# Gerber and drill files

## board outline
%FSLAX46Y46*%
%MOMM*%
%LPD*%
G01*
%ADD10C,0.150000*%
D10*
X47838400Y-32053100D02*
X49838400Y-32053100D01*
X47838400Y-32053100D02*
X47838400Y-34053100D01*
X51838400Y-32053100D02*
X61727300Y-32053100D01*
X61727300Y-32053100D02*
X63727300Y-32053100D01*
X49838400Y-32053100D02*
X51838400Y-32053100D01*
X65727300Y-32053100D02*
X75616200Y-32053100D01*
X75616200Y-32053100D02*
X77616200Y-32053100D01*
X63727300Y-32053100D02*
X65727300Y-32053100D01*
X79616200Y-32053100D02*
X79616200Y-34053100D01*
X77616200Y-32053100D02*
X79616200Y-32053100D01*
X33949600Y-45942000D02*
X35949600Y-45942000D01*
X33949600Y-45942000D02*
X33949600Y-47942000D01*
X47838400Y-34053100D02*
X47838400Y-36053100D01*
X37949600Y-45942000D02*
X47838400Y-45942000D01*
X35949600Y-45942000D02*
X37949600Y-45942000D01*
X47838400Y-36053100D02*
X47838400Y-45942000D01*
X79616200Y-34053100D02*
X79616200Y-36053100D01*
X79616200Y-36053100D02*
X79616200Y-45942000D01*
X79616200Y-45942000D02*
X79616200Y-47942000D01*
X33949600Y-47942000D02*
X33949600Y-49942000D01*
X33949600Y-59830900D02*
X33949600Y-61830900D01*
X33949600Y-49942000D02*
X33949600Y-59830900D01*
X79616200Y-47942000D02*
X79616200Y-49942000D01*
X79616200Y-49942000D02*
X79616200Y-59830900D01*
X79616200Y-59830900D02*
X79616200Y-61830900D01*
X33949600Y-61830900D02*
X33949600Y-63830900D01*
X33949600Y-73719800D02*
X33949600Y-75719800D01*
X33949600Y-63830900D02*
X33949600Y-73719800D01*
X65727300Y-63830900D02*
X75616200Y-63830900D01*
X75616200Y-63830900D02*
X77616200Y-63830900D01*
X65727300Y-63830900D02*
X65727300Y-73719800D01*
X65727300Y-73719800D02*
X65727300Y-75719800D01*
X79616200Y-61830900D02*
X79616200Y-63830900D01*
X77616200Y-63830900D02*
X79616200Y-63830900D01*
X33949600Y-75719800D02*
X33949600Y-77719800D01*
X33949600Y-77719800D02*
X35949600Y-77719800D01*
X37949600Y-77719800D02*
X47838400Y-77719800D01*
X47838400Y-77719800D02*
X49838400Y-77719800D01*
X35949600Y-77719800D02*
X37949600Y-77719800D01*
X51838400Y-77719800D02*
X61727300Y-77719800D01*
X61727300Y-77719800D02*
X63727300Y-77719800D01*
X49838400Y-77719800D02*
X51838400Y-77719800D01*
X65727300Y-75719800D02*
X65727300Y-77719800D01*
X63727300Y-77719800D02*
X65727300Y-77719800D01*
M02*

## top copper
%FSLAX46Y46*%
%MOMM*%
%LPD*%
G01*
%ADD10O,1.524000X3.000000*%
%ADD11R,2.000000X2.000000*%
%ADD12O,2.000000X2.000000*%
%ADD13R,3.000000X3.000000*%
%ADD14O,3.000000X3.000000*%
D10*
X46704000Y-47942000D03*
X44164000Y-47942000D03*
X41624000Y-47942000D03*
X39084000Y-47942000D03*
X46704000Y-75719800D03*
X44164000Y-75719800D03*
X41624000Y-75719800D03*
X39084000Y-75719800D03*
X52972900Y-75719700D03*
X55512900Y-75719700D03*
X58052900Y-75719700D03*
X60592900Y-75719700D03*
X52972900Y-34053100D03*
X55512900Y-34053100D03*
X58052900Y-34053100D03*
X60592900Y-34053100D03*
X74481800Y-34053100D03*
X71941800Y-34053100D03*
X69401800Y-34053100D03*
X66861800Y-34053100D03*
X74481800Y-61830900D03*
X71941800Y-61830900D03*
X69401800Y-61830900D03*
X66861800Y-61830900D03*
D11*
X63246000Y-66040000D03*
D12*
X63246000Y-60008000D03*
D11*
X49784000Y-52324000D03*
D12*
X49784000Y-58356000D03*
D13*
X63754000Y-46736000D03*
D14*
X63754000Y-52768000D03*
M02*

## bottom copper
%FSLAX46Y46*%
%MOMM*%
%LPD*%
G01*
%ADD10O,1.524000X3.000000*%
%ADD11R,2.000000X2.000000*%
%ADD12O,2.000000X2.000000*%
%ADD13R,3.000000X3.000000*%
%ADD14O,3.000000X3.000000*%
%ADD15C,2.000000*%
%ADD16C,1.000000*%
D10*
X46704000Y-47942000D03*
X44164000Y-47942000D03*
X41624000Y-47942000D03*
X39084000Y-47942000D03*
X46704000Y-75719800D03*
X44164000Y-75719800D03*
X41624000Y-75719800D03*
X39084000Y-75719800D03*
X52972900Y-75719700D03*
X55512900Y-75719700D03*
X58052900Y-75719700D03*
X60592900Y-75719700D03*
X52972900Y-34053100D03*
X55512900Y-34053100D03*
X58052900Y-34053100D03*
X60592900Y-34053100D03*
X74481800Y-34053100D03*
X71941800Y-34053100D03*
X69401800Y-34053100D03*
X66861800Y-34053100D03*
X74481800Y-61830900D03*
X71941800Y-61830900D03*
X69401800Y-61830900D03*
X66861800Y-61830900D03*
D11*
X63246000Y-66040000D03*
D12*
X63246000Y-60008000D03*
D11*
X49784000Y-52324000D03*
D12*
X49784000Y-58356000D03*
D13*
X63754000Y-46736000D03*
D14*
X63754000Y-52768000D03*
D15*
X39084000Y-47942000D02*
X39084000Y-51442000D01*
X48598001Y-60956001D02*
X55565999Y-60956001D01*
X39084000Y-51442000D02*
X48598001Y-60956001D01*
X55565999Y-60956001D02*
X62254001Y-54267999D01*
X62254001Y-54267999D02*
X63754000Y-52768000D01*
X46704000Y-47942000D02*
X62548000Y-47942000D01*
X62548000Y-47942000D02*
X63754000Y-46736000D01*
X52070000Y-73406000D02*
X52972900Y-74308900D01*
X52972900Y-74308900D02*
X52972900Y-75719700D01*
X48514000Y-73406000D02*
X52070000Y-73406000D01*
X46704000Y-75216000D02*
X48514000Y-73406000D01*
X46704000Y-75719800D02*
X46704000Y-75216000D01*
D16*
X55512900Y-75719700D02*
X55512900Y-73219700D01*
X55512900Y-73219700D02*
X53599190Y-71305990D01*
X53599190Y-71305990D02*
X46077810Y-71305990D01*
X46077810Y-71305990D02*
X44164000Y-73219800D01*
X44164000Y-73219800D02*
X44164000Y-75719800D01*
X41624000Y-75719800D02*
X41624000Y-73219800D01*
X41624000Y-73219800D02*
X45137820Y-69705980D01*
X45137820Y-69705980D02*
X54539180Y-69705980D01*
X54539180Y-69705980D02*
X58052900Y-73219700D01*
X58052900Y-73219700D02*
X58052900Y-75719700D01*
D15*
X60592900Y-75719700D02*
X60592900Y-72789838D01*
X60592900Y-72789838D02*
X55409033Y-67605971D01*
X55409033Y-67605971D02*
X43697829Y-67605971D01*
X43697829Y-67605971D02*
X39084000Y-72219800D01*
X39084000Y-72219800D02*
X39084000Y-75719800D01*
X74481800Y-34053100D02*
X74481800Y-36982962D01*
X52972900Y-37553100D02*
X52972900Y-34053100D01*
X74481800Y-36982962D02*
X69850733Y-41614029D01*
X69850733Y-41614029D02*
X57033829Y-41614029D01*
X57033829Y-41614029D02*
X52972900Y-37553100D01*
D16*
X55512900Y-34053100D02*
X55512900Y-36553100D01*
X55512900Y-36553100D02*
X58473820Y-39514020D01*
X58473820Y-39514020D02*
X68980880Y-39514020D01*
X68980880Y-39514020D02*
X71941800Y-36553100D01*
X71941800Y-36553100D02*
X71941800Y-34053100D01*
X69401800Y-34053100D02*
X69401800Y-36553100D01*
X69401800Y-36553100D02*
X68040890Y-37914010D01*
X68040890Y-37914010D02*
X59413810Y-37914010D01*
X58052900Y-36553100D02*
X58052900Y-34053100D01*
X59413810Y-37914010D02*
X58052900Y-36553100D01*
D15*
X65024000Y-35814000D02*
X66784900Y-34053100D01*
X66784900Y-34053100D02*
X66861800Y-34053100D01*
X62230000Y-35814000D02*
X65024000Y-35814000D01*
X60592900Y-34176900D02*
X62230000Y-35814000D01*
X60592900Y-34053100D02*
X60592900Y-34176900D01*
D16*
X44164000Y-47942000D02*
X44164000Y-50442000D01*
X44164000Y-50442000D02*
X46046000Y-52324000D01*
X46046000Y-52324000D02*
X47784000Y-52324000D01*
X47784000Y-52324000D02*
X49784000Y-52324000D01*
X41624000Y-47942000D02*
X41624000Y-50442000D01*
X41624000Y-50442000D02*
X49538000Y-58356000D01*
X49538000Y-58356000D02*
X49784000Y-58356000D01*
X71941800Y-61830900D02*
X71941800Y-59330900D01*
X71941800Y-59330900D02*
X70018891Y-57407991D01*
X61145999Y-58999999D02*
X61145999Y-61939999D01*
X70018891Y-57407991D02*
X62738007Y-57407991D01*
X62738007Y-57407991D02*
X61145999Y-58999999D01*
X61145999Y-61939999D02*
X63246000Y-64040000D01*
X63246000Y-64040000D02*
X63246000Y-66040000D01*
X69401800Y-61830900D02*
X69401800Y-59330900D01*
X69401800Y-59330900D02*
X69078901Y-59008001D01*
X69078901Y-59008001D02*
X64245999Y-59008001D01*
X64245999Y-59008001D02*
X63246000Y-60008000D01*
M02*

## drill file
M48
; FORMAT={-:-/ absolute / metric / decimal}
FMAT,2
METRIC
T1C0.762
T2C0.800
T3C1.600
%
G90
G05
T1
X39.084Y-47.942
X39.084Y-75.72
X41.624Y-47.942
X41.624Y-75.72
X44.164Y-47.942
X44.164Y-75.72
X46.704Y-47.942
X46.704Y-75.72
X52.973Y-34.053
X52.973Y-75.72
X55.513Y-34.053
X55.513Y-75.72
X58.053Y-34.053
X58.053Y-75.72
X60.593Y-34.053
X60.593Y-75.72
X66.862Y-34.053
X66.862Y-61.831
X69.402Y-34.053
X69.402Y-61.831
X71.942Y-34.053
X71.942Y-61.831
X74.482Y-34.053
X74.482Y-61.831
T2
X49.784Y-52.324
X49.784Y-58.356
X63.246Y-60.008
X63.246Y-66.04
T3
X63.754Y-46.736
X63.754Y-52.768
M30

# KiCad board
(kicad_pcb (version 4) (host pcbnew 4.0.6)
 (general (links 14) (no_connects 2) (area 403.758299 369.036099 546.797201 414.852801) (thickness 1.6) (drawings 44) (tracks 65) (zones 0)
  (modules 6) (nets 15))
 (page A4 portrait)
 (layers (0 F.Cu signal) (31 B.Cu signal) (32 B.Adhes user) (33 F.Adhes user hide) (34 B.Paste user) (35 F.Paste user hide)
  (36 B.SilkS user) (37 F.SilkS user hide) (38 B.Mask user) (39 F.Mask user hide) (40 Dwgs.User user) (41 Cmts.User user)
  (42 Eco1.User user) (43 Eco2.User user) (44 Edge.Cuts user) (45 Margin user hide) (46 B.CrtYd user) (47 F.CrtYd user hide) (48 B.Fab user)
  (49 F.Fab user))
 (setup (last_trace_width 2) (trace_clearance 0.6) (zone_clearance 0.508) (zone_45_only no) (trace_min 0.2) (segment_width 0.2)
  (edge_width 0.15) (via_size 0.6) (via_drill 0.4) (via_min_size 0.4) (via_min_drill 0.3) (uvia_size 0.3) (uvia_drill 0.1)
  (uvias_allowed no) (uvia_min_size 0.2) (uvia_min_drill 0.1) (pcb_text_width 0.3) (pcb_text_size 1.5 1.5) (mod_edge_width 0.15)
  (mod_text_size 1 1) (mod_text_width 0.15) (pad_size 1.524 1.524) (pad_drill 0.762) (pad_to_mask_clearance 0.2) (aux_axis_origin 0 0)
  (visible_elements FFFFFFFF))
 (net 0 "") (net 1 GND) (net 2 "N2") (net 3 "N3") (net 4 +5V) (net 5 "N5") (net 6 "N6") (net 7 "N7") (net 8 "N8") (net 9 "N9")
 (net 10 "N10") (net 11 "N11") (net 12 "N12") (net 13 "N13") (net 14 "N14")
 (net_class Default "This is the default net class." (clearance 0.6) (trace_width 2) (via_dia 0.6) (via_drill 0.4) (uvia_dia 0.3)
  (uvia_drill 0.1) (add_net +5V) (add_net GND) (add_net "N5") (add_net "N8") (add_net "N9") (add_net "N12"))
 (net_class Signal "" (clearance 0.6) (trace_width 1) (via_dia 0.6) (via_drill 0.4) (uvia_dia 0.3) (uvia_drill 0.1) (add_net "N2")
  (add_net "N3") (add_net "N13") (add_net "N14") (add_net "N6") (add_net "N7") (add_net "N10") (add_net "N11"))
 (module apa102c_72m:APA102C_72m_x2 (layer B.Cu) (at 42.894 61.8309 270)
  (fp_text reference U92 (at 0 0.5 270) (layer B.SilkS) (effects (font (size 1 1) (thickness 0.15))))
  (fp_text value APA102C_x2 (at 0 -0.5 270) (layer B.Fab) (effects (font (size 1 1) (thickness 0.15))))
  (pad 1 thru_hole oval (at -13.8889 -3.81 270) (size 3 1.524) (drill 0.762) (layers *.Cu *.Mask) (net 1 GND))
  (pad 2 thru_hole oval (at -13.8889 -1.27 270) (size 3 1.524) (drill 0.762) (layers *.Cu *.Mask) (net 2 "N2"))
  (pad 3 thru_hole oval (at -13.8889 1.27 270) (size 3 1.524) (drill 0.762) (layers *.Cu *.Mask) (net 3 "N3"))
  (pad 4 thru_hole oval (at -13.8889 3.81 270) (size 3 1.524) (drill 0.762) (layers *.Cu *.Mask) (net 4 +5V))
  (pad 5 thru_hole oval (at 13.8889 -3.81 270) (size 3 1.524) (drill 0.762) (layers *.Cu *.Mask) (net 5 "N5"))
  (pad 6 thru_hole oval (at 13.8889 -1.27 270) (size 3 1.524) (drill 0.762) (layers *.Cu *.Mask) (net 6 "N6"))
  (pad 7 thru_hole oval (at 13.8889 1.27 270) (size 3 1.524) (drill 0.762) (layers *.Cu *.Mask) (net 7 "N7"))
  (pad 8 thru_hole oval (at 13.8889 3.81 270) (size 3 1.524) (drill 0.762) (layers *.Cu *.Mask) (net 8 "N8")))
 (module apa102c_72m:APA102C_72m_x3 (layer B.Cu) (at 56.7829 54.8864 90)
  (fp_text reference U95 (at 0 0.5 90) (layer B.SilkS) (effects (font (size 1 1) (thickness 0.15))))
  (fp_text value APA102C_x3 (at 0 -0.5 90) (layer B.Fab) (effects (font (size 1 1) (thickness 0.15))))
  (pad 1 thru_hole oval (at -20.8333 -3.81 90) (size 3 1.524) (drill 0.762) (layers *.Cu *.Mask) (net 5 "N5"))
  (pad 2 thru_hole oval (at -20.8333 -1.27 90) (size 3 1.524) (drill 0.762) (layers *.Cu *.Mask) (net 6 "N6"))
  (pad 3 thru_hole oval (at -20.8333 1.27 90) (size 3 1.524) (drill 0.762) (layers *.Cu *.Mask) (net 7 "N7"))
  (pad 4 thru_hole oval (at -20.8333 3.81 90) (size 3 1.524) (drill 0.762) (layers *.Cu *.Mask) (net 8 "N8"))
  (pad 5 thru_hole oval (at 20.8333 -3.81 90) (size 3 1.524) (drill 0.762) (layers *.Cu *.Mask) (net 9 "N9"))
  (pad 6 thru_hole oval (at 20.8333 -1.27 90) (size 3 1.524) (drill 0.762) (layers *.Cu *.Mask) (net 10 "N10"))
  (pad 7 thru_hole oval (at 20.8333 1.27 90) (size 3 1.524) (drill 0.762) (layers *.Cu *.Mask) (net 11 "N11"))
  (pad 8 thru_hole oval (at 20.8333 3.81 90) (size 3 1.524) (drill 0.762) (layers *.Cu *.Mask) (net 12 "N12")))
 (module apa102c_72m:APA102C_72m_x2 (layer B.Cu) (at 70.6718 47.942 270)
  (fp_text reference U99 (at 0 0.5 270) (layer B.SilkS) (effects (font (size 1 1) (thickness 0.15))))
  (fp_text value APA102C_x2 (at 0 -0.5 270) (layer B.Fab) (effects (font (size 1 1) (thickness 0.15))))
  (pad 1 thru_hole oval (at -13.8889 -3.81 270) (size 3 1.524) (drill 0.762) (layers *.Cu *.Mask) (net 9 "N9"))
  (pad 2 thru_hole oval (at -13.8889 -1.27 270) (size 3 1.524) (drill 0.762) (layers *.Cu *.Mask) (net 10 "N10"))
  (pad 3 thru_hole oval (at -13.8889 1.27 270) (size 3 1.524) (drill 0.762) (layers *.Cu *.Mask) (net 11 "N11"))
  (pad 4 thru_hole oval (at -13.8889 3.81 270) (size 3 1.524) (drill 0.762) (layers *.Cu *.Mask) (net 12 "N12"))
  (pad 5 thru_hole oval (at 13.8889 -3.81 270) (size 3 1.524) (drill 0.762) (layers *.Cu *.Mask))
  (pad 6 thru_hole oval (at 13.8889 -1.27 270) (size 3 1.524) (drill 0.762) (layers *.Cu *.Mask) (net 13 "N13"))
  (pad 7 thru_hole oval (at 13.8889 1.27 270) (size 3 1.524) (drill 0.762) (layers *.Cu *.Mask) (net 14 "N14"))
  (pad 8 thru_hole oval (at 13.8889 3.81 270) (size 3 1.524) (drill 0.762) (layers *.Cu *.Mask)))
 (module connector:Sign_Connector (layer F.Cu) (at 63.246 64.008 180)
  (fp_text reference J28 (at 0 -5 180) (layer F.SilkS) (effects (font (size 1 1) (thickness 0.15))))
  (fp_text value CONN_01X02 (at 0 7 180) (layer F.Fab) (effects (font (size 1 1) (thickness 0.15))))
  (pad 1 thru_hole rect (at 0 -2.032 180) (size 2 2) (drill 0.8) (layers *.Cu *.Mask) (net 13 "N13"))
  (pad 2 thru_hole oval (at 0 4 180) (size 2 2) (drill 0.8) (layers *.Cu *.Mask) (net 14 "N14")))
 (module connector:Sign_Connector (layer F.Cu) (at 49.784 54.356)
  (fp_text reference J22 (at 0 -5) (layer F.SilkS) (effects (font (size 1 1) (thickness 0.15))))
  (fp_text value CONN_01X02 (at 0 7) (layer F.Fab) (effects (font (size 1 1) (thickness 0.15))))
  (pad 1 thru_hole rect (at 0 -2.032) (size 2 2) (drill 0.8) (layers *.Cu *.Mask) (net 2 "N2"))
  (pad 2 thru_hole oval (at 0 4) (size 2 2) (drill 0.8) (layers *.Cu *.Mask) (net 3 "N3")))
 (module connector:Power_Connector (layer F.Cu) (at 63.754 48.768)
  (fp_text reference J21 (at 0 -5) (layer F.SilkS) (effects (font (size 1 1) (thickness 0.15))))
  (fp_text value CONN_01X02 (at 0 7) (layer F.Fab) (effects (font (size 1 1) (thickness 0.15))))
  (pad 1 thru_hole rect (at 0 -2.032) (size 3 3) (drill 1.6) (layers *.Cu *.Mask) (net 1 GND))
  (pad 2 thru_hole oval (at 0 4) (size 3 3) (drill 1.6) (layers *.Cu *.Mask) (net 4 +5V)))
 (gr_line (start 47.8384 32.0531) (end 49.8384 32.0531) (layer Edge.Cuts) (width 0.15))
 (gr_line (start 47.8384 32.0531) (end 47.8384 34.0531) (layer Edge.Cuts) (width 0.15))
 (gr_line (start 51.8384 32.0531) (end 61.7273 32.0531) (layer Edge.Cuts) (width 0.15))
 (gr_line (start 61.7273 32.0531) (end 63.7273 32.0531) (layer Edge.Cuts) (width 0.15))
 (gr_line (start 49.8384 32.0531) (end 51.8384 32.0531) (layer Edge.Cuts) (width 0.15))
 (gr_line (start 65.7273 32.0531) (end 75.6162 32.0531) (layer Edge.Cuts) (width 0.15))
 (gr_line (start 75.6162 32.0531) (end 77.6162 32.0531) (layer Edge.Cuts) (width 0.15))
 (gr_line (start 63.7273 32.0531) (end 65.7273 32.0531) (layer Edge.Cuts) (width 0.15))
 (gr_line (start 79.6162 32.0531) (end 79.6162 34.0531) (layer Edge.Cuts) (width 0.15))
 (gr_line (start 77.6162 32.0531) (end 79.6162 32.0531) (layer Edge.Cuts) (width 0.15))
 (gr_line (start 33.9496 45.942) (end 35.9496 45.942) (layer Edge.Cuts) (width 0.15))
 (gr_line (start 33.9496 45.942) (end 33.9496 47.942) (layer Edge.Cuts) (width 0.15))
 (gr_line (start 47.8384 34.0531) (end 47.8384 36.0531) (layer Edge.Cuts) (width 0.15))
 (gr_line (start 37.9496 45.942) (end 47.8384 45.942) (layer Edge.Cuts) (width 0.15))
 (gr_line (start 35.9496 45.942) (end 37.9496 45.942) (layer Edge.Cuts) (width 0.15))
 (gr_line (start 47.8384 36.0531) (end 47.8384 45.942) (layer Edge.Cuts) (width 0.15))
 (gr_line (start 79.6162 34.0531) (end 79.6162 36.0531) (layer Edge.Cuts) (width 0.15))
 (gr_line (start 79.6162 36.0531) (end 79.6162 45.942) (layer Edge.Cuts) (width 0.15))
 (gr_line (start 79.6162 45.942) (end 79.6162 47.942) (layer Edge.Cuts) (width 0.15))
 (gr_line (start 33.9496 47.942) (end 33.9496 49.942) (layer Edge.Cuts) (width 0.15))
 (gr_line (start 33.9496 59.8309) (end 33.9496 61.8309) (layer Edge.Cuts) (width 0.15))
 (gr_line (start 33.9496 49.942) (end 33.9496 59.8309) (layer Edge.Cuts) (width 0.15))
 (gr_line (start 79.6162 47.942) (end 79.6162 49.942) (layer Edge.Cuts) (width 0.15))
 (gr_line (start 79.6162 49.942) (end 79.6162 59.8309) (layer Edge.Cuts) (width 0.15))
 (gr_line (start 79.6162 59.8309) (end 79.6162 61.8309) (layer Edge.Cuts) (width 0.15))
 (gr_line (start 33.9496 61.8309) (end 33.9496 63.8309) (layer Edge.Cuts) (width 0.15))
 (gr_line (start 33.9496 73.7198) (end 33.9496 75.7198) (layer Edge.Cuts) (width 0.15))
 (gr_line (start 33.9496 63.8309) (end 33.9496 73.7198) (layer Edge.Cuts) (width 0.15))
 (gr_line (start 65.7273 63.8309) (end 75.6162 63.8309) (layer Edge.Cuts) (width 0.15))
 (gr_line (start 75.6162 63.8309) (end 77.6162 63.8309) (layer Edge.Cuts) (width 0.15))
 (gr_line (start 65.7273 63.8309) (end 65.7273 73.7198) (layer Edge.Cuts) (width 0.15))
 (gr_line (start 65.7273 73.7198) (end 65.7273 75.7198) (layer Edge.Cuts) (width 0.15))
 (gr_line (start 79.6162 61.8309) (end 79.6162 63.8309) (layer Edge.Cuts) (width 0.15))
 (gr_line (start 77.6162 63.8309) (end 79.6162 63.8309) (layer Edge.Cuts) (width 0.15))
 (gr_line (start 33.9496 75.7198) (end 33.9496 77.7198) (layer Edge.Cuts) (width 0.15))
 (gr_line (start 33.9496 77.7198) (end 35.9496 77.7198) (layer Edge.Cuts) (width 0.15))
 (gr_line (start 37.9496 77.7198) (end 47.8384 77.7198) (layer Edge.Cuts) (width 0.15))
 (gr_line (start 47.8384 77.7198) (end 49.8384 77.7198) (layer Edge.Cuts) (width 0.15))
 (gr_line (start 35.9496 77.7198) (end 37.9496 77.7198) (layer Edge.Cuts) (width 0.15))
 (gr_line (start 51.8384 77.7198) (end 61.7273 77.7198) (layer Edge.Cuts) (width 0.15))
 (gr_line (start 61.7273 77.7198) (end 63.7273 77.7198) (layer Edge.Cuts) (width 0.15))
 (gr_line (start 49.8384 77.7198) (end 51.8384 77.7198) (layer Edge.Cuts) (width 0.15))
 (gr_line (start 65.7273 75.7198) (end 65.7273 77.7198) (layer Edge.Cuts) (width 0.15))
 (gr_line (start 63.7273 77.7198) (end 65.7273 77.7198) (layer Edge.Cuts) (width 0.15))
 (segment (start 39.084 47.942) (end 39.084 51.442) (width 2) (layer B.Cu) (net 4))
 (segment (start 48.598001 60.956001) (end 55.565999 60.956001) (width 2) (layer B.Cu) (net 4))
 (segment (start 39.084 51.442) (end 48.598001 60.956001) (width 2) (layer B.Cu) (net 4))
 (segment (start 55.565999 60.956001) (end 62.254001 54.267999) (width 2) (layer B.Cu) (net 4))
 (segment (start 62.254001 54.267999) (end 63.754 52.768) (width 2) (layer B.Cu) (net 4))
 (segment (start 46.704 47.942) (end 62.548 47.942) (width 2) (layer B.Cu) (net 1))
 (segment (start 62.548 47.942) (end 63.754 46.736) (width 2) (layer B.Cu) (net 1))
 (segment (start 52.07 73.406) (end 52.9729 74.3089) (width 2) (layer B.Cu) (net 5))
 (segment (start 52.9729 74.3089) (end 52.9729 75.7197) (width 2) (layer B.Cu) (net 5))
 (segment (start 48.514 73.406) (end 52.07 73.406) (width 2) (layer B.Cu) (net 5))
 (segment (start 46.704 75.216) (end 48.514 73.406) (width 2) (layer B.Cu) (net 5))
 (segment (start 46.704 75.7198) (end 46.704 75.216) (width 2) (layer B.Cu) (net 5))
 (segment (start 55.5129 75.7197) (end 55.5129 73.2197) (width 1) (layer B.Cu) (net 6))
 (segment (start 55.5129 73.2197) (end 53.59919 71.30599) (width 1) (layer B.Cu) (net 6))
 (segment (start 53.59919 71.30599) (end 46.07781 71.30599) (width 1) (layer B.Cu) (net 6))
 (segment (start 46.07781 71.30599) (end 44.164 73.2198) (width 1) (layer B.Cu) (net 6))
 (segment (start 44.164 73.2198) (end 44.164 75.7198) (width 1) (layer B.Cu) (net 6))
 (segment (start 41.624 75.7198) (end 41.624 73.2198) (width 1) (layer B.Cu) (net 7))
 (segment (start 41.624 73.2198) (end 45.13782 69.70598) (width 1) (layer B.Cu) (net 7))
 (segment (start 45.13782 69.70598) (end 54.53918 69.70598) (width 1) (layer B.Cu) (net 7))
 (segment (start 54.53918 69.70598) (end 58.0529 73.2197) (width 1) (layer B.Cu) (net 7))
 (segment (start 58.0529 73.2197) (end 58.0529 75.7197) (width 1) (layer B.Cu) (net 7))
 (segment (start 60.5929 75.7197) (end 60.5929 72.789838) (width 2) (layer B.Cu) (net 8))
 (segment (start 60.5929 72.789838) (end 55.409033 67.605971) (width 2) (layer B.Cu) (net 8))
 (segment (start 55.409033 67.605971) (end 43.697829 67.605971) (width 2) (layer B.Cu) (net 8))
 (segment (start 43.697829 67.605971) (end 39.084 72.2198) (width 2) (layer B.Cu) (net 8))
 (segment (start 39.084 72.2198) (end 39.084 75.7198) (width 2) (layer B.Cu) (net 8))
 (segment (start 74.4818 34.0531) (end 74.4818 36.982962) (width 2) (layer B.Cu) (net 9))
 (segment (start 52.9729 37.5531) (end 52.9729 34.0531) (width 2) (layer B.Cu) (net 9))
 (segment (start 74.4818 36.982962) (end 69.850733 41.614029) (width 2) (layer B.Cu) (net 9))
 (segment (start 69.850733 41.614029) (end 57.033829 41.614029) (width 2) (layer B.Cu) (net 9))
 (segment (start 57.033829 41.614029) (end 52.9729 37.5531) (width 2) (layer B.Cu) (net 9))
 (segment (start 55.5129 34.0531) (end 55.5129 36.5531) (width 1) (layer B.Cu) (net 10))
 (segment (start 55.5129 36.5531) (end 58.47382 39.51402) (width 1) (layer B.Cu) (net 10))
 (segment (start 58.47382 39.51402) (end 68.98088 39.51402) (width 1) (layer B.Cu) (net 10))
 (segment (start 68.98088 39.51402) (end 71.9418 36.5531) (width 1) (layer B.Cu) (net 10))
 (segment (start 71.9418 36.5531) (end 71.9418 34.0531) (width 1) (layer B.Cu) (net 10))
 (segment (start 69.4018 34.0531) (end 69.4018 36.5531) (width 1) (layer B.Cu) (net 11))
 (segment (start 69.4018 36.5531) (end 68.04089 37.91401) (width 1) (layer B.Cu) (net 11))
 (segment (start 68.04089 37.91401) (end 59.41381 37.91401) (width 1) (layer B.Cu) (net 11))
 (segment (start 58.0529 36.5531) (end 58.0529 34.0531) (width 1) (layer B.Cu) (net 11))
 (segment (start 59.41381 37.91401) (end 58.0529 36.5531) (width 1) (layer B.Cu) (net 11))
 (segment (start 65.024 35.814) (end 66.7849 34.0531) (width 2) (layer B.Cu) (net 12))
 (segment (start 66.7849 34.0531) (end 66.8618 34.0531) (width 2) (layer B.Cu) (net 12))
 (segment (start 62.23 35.814) (end 65.024 35.814) (width 2) (layer B.Cu) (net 12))
 (segment (start 60.5929 34.1769) (end 62.23 35.814) (width 2) (layer B.Cu) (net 12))
 (segment (start 60.5929 34.0531) (end 60.5929 34.1769) (width 2) (layer B.Cu) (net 12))
 (segment (start 44.164 47.942) (end 44.164 50.442) (width 1) (layer B.Cu) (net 2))
 (segment (start 44.164 50.442) (end 46.046 52.324) (width 1) (layer B.Cu) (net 2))
 (segment (start 46.046 52.324) (end 47.784 52.324) (width 1) (layer B.Cu) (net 2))
 (segment (start 47.784 52.324) (end 49.784 52.324) (width 1) (layer B.Cu) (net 2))
 (segment (start 41.624 47.942) (end 41.624 50.442) (width 1) (layer B.Cu) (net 3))
 (segment (start 41.624 50.442) (end 49.538 58.356) (width 1) (layer B.Cu) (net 3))
 (segment (start 49.538 58.356) (end 49.784 58.356) (width 1) (layer B.Cu) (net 3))
 (segment (start 71.9418 61.8309) (end 71.9418 59.3309) (width 1) (layer B.Cu) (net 13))
 (segment (start 71.9418 59.3309) (end 70.018891 57.407991) (width 1) (layer B.Cu) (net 13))
 (segment (start 61.145999 58.999999) (end 61.145999 61.939999) (width 1) (layer B.Cu) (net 13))
 (segment (start 70.018891 57.407991) (end 62.738007 57.407991) (width 1) (layer B.Cu) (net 13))
 (segment (start 62.738007 57.407991) (end 61.145999 58.999999) (width 1) (layer B.Cu) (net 13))
 (segment (start 61.145999 61.939999) (end 63.246 64.04) (width 1) (layer B.Cu) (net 13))
 (segment (start 63.246 64.04) (end 63.246 66.04) (width 1) (layer B.Cu) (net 13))
 (segment (start 69.4018 61.8309) (end 69.4018 59.3309) (width 1) (layer B.Cu) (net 14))
 (segment (start 69.4018 59.3309) (end 69.078901 59.008001) (width 1) (layer B.Cu) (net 14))
 (segment (start 69.078901 59.008001) (end 64.245999 59.008001) (width 1) (layer B.Cu) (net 14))
 (segment (start 64.245999 59.008001) (end 63.246 60.008) (width 1) (layer B.Cu) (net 14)))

